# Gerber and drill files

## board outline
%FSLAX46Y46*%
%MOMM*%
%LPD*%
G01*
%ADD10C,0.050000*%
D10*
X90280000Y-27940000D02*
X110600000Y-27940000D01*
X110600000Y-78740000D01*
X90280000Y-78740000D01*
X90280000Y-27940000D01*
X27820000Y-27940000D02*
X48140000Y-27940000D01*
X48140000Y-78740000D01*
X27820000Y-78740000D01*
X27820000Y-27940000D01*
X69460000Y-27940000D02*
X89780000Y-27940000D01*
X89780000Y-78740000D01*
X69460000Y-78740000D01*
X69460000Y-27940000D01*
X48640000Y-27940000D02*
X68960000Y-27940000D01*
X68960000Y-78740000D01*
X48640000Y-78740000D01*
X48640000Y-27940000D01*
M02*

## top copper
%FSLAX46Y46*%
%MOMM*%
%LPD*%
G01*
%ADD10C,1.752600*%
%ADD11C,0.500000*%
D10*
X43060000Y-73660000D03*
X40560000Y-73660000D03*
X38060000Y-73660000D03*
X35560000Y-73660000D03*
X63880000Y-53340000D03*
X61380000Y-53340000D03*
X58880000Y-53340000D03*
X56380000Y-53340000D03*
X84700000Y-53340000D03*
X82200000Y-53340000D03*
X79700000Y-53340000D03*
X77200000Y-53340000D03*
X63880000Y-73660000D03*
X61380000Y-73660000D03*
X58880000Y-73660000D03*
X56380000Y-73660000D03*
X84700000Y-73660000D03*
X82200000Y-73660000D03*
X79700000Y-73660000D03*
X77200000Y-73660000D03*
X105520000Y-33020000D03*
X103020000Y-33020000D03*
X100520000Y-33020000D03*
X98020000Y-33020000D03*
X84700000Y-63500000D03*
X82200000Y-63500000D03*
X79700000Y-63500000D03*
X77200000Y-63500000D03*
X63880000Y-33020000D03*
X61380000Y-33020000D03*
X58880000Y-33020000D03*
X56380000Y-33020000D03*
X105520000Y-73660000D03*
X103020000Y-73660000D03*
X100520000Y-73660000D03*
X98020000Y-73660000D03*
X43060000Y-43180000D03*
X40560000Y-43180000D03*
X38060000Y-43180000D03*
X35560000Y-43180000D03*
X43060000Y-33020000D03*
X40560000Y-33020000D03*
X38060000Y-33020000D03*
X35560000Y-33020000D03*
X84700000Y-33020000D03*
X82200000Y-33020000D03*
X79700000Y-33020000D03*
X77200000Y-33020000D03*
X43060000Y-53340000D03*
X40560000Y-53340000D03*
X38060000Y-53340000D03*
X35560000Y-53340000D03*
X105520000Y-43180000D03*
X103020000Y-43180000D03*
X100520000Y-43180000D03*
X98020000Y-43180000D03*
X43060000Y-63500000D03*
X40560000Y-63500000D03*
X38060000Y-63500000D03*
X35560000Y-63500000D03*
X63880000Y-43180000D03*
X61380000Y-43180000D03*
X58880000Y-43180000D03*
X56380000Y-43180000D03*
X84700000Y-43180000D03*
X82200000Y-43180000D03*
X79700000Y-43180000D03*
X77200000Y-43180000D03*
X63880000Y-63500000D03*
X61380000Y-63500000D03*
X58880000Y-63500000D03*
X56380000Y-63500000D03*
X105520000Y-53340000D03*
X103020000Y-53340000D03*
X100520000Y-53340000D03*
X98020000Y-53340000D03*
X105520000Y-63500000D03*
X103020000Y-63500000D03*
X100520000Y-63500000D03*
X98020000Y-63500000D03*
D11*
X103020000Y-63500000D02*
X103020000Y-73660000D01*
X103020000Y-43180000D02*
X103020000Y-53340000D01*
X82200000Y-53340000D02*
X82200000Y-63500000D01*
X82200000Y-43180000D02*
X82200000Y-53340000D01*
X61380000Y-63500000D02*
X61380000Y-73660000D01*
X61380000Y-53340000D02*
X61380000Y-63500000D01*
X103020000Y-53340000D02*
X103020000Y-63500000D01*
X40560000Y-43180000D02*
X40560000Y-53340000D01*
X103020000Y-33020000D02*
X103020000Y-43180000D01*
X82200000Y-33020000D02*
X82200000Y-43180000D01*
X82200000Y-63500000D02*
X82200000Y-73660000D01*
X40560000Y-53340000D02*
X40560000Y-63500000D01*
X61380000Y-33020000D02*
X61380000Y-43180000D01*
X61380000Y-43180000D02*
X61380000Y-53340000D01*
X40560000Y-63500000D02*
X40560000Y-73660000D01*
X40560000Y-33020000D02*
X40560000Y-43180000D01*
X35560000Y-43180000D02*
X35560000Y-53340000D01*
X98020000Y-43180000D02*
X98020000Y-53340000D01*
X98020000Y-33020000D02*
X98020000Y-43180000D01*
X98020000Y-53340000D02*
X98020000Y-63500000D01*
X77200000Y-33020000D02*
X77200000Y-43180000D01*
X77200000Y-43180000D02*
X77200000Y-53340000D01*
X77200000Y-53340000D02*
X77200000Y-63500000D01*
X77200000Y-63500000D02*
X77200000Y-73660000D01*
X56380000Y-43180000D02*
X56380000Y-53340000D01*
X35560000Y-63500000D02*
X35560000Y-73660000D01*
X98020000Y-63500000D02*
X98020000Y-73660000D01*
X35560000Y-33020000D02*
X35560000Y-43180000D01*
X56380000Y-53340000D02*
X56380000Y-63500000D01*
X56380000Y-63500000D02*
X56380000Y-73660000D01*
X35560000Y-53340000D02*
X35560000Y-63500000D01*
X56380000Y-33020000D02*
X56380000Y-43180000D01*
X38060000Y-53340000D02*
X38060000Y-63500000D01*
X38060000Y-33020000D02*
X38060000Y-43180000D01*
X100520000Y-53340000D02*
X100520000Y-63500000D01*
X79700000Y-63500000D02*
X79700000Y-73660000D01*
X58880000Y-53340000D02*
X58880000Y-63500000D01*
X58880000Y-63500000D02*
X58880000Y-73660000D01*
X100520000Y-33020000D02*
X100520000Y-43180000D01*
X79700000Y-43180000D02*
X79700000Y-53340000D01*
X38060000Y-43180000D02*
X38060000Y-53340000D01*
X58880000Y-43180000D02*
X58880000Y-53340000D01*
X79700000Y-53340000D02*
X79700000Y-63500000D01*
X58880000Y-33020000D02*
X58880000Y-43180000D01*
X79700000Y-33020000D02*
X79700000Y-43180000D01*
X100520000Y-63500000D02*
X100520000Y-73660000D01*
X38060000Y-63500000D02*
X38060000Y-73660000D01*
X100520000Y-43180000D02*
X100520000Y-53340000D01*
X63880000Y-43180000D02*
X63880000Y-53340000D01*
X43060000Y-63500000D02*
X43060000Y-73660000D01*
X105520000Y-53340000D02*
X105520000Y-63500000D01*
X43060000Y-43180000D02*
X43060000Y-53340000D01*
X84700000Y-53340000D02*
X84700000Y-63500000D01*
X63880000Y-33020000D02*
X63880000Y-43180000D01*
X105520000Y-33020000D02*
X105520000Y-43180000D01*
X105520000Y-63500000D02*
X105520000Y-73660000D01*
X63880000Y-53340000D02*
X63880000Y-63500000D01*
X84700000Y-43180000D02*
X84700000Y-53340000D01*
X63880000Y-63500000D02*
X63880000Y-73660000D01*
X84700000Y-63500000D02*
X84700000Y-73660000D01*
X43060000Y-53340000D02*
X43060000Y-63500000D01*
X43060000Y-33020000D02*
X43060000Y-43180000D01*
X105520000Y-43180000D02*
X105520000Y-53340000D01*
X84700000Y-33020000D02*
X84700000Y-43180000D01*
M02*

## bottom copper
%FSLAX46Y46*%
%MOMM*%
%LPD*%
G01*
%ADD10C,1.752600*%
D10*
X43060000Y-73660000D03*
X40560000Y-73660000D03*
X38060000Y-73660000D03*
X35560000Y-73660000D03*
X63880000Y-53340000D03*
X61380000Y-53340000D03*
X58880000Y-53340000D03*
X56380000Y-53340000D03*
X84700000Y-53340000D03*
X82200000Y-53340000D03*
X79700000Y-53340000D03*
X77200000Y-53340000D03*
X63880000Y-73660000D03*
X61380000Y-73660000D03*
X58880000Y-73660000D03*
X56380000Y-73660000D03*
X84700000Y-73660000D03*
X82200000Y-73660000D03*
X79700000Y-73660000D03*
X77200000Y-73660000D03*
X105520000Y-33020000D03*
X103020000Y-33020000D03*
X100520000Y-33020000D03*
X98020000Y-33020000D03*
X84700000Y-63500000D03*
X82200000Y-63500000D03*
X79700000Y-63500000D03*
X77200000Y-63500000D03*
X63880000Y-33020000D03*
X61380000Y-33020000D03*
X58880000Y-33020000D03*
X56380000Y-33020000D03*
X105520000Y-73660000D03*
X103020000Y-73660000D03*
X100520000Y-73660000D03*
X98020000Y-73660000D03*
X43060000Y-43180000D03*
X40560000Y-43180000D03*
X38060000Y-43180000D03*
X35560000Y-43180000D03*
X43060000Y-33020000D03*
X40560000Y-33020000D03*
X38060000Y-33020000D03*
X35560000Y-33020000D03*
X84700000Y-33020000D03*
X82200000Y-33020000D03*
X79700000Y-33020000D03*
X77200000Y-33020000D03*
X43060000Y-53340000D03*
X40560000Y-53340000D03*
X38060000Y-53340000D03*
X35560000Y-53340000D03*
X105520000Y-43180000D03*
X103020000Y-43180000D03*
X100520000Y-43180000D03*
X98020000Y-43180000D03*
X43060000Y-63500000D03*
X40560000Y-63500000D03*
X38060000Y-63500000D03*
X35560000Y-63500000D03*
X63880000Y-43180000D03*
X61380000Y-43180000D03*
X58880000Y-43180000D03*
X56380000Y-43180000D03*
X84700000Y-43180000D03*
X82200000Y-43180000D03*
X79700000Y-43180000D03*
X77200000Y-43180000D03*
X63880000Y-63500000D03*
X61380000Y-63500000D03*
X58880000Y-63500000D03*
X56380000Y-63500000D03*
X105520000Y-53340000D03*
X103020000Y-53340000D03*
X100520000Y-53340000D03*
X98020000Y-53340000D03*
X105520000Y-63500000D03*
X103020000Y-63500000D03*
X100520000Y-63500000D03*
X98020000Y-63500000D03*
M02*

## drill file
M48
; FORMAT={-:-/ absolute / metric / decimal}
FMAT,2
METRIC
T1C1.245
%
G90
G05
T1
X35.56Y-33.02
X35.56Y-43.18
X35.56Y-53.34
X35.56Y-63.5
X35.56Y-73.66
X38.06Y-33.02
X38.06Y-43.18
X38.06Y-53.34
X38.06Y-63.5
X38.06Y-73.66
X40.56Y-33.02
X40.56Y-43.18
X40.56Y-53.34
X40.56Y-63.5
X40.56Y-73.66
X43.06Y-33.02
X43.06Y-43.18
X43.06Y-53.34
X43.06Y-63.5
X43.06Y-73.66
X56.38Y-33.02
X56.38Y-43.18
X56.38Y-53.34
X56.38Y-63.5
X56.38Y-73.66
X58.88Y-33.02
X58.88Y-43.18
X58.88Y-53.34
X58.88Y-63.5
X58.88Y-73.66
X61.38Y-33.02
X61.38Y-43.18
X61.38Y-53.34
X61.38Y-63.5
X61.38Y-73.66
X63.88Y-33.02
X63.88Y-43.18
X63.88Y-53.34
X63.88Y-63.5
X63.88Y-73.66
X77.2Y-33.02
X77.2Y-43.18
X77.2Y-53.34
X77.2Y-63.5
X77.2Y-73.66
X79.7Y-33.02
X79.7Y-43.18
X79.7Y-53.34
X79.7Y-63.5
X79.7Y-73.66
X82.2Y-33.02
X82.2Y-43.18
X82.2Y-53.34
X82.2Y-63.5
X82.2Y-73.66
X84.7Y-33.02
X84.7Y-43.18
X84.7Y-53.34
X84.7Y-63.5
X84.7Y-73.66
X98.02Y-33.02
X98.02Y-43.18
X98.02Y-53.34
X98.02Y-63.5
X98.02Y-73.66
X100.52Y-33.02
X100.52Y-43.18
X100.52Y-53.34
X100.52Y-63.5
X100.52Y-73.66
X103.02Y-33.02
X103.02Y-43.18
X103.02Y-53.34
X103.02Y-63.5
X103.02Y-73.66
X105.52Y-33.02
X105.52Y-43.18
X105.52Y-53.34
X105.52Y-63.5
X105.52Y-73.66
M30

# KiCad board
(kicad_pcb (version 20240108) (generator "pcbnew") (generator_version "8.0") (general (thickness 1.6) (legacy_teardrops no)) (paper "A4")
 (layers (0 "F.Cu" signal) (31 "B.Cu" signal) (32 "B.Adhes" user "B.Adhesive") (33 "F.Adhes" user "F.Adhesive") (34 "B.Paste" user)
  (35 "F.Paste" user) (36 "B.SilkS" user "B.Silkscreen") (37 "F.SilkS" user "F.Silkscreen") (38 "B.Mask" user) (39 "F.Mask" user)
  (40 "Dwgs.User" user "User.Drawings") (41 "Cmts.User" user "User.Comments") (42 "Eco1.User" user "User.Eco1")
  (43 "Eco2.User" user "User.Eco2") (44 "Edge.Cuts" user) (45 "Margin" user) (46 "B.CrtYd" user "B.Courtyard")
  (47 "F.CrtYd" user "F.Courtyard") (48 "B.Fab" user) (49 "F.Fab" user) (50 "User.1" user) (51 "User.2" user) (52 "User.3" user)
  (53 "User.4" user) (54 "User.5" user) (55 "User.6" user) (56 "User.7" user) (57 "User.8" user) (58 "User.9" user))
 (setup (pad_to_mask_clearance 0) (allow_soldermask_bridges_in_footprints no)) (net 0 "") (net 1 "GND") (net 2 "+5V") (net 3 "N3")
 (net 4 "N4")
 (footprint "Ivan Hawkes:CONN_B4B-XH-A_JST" (layer "F.Cu") (at 43.06 73.66)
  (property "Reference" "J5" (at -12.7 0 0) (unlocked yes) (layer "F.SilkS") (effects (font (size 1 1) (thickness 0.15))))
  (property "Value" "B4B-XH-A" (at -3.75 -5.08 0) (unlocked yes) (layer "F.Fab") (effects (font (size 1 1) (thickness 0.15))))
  (pad "1" thru_hole circle (at 0 0) (size 1.7526 1.7526) (drill 1.2446) (layers "*.Cu" "*.Mask") (remove_unused_layers no) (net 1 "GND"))
  (pad "2" thru_hole circle (at -2.5 0) (size 1.7526 1.7526) (drill 1.2446) (layers "*.Cu" "*.Mask") (remove_unused_layers no) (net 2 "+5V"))
  (pad "3" thru_hole circle (at -5 0) (size 1.7526 1.7526) (drill 1.2446) (layers "*.Cu" "*.Mask") (remove_unused_layers no) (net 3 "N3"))
  (pad "4" thru_hole circle (at -7.5 0) (size 1.7526 1.7526) (drill 1.2446) (layers "*.Cu" "*.Mask") (remove_unused_layers no) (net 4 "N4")))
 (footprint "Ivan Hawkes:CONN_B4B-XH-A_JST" (layer "F.Cu") (at 63.88 53.34)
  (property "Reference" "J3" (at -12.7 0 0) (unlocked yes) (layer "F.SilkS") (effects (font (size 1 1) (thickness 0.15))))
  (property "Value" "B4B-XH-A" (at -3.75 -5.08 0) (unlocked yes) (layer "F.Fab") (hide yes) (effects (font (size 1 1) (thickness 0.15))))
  (pad "1" thru_hole circle (at 0 0) (size 1.7526 1.7526) (drill 1.2446) (layers "*.Cu" "*.Mask") (remove_unused_layers no) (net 1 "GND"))
  (pad "2" thru_hole circle (at -2.5 0) (size 1.7526 1.7526) (drill 1.2446) (layers "*.Cu" "*.Mask") (remove_unused_layers no) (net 2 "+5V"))
  (pad "3" thru_hole circle (at -5 0) (size 1.7526 1.7526) (drill 1.2446) (layers "*.Cu" "*.Mask") (remove_unused_layers no) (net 3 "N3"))
  (pad "4" thru_hole circle (at -7.5 0) (size 1.7526 1.7526) (drill 1.2446) (layers "*.Cu" "*.Mask") (remove_unused_layers no) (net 4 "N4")))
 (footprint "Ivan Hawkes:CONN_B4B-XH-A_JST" (layer "F.Cu") (at 84.7 53.34)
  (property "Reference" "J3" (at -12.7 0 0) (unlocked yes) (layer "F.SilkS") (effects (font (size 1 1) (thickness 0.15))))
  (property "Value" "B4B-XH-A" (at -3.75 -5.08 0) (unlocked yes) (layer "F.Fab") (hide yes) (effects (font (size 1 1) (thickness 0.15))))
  (pad "1" thru_hole circle (at 0 0) (size 1.7526 1.7526) (drill 1.2446) (layers "*.Cu" "*.Mask") (remove_unused_layers no) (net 1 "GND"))
  (pad "2" thru_hole circle (at -2.5 0) (size 1.7526 1.7526) (drill 1.2446) (layers "*.Cu" "*.Mask") (remove_unused_layers no) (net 2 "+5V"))
  (pad "3" thru_hole circle (at -5 0) (size 1.7526 1.7526) (drill 1.2446) (layers "*.Cu" "*.Mask") (remove_unused_layers no) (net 3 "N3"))
  (pad "4" thru_hole circle (at -7.5 0) (size 1.7526 1.7526) (drill 1.2446) (layers "*.Cu" "*.Mask") (remove_unused_layers no) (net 4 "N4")))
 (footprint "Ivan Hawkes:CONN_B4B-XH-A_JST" (layer "F.Cu") (at 63.88 73.66)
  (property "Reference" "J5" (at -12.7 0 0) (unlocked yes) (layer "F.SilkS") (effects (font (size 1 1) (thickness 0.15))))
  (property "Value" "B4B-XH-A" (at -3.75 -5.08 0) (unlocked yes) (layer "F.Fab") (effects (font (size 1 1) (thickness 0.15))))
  (pad "1" thru_hole circle (at 0 0) (size 1.7526 1.7526) (drill 1.2446) (layers "*.Cu" "*.Mask") (remove_unused_layers no) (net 1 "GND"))
  (pad "2" thru_hole circle (at -2.5 0) (size 1.7526 1.7526) (drill 1.2446) (layers "*.Cu" "*.Mask") (remove_unused_layers no) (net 2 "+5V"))
  (pad "3" thru_hole circle (at -5 0) (size 1.7526 1.7526) (drill 1.2446) (layers "*.Cu" "*.Mask") (remove_unused_layers no) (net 3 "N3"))
  (pad "4" thru_hole circle (at -7.5 0) (size 1.7526 1.7526) (drill 1.2446) (layers "*.Cu" "*.Mask") (remove_unused_layers no) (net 4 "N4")))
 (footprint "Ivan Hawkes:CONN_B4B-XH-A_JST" (layer "F.Cu") (at 84.7 73.66)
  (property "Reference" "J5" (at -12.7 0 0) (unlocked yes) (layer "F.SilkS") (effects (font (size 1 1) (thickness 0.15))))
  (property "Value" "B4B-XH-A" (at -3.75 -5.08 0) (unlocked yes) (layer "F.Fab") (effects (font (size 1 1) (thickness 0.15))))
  (pad "1" thru_hole circle (at 0 0) (size 1.7526 1.7526) (drill 1.2446) (layers "*.Cu" "*.Mask") (remove_unused_layers no) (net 1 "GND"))
  (pad "2" thru_hole circle (at -2.5 0) (size 1.7526 1.7526) (drill 1.2446) (layers "*.Cu" "*.Mask") (remove_unused_layers no) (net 2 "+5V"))
  (pad "3" thru_hole circle (at -5 0) (size 1.7526 1.7526) (drill 1.2446) (layers "*.Cu" "*.Mask") (remove_unused_layers no) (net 3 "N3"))
  (pad "4" thru_hole circle (at -7.5 0) (size 1.7526 1.7526) (drill 1.2446) (layers "*.Cu" "*.Mask") (remove_unused_layers no) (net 4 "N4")))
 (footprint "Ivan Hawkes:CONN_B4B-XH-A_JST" (layer "F.Cu") (at 105.52 33.02)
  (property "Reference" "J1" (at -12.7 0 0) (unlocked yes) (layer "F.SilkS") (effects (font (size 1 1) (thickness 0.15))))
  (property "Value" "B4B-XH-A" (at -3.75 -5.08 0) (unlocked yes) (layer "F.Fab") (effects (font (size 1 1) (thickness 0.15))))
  (pad "1" thru_hole circle (at 0 0) (size 1.7526 1.7526) (drill 1.2446) (layers "*.Cu" "*.Mask") (remove_unused_layers no) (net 1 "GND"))
  (pad "2" thru_hole circle (at -2.5 0) (size 1.7526 1.7526) (drill 1.2446) (layers "*.Cu" "*.Mask") (remove_unused_layers no) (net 2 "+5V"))
  (pad "3" thru_hole circle (at -5 0) (size 1.7526 1.7526) (drill 1.2446) (layers "*.Cu" "*.Mask") (remove_unused_layers no) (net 3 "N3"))
  (pad "4" thru_hole circle (at -7.5 0) (size 1.7526 1.7526) (drill 1.2446) (layers "*.Cu" "*.Mask") (remove_unused_layers no) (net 4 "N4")))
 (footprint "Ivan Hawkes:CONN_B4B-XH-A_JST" (layer "F.Cu") (at 84.7 63.5)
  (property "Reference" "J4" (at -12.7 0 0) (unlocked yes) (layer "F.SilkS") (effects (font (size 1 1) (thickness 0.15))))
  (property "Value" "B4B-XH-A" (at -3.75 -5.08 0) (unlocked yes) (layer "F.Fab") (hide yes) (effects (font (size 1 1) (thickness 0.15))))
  (pad "1" thru_hole circle (at 0 0) (size 1.7526 1.7526) (drill 1.2446) (layers "*.Cu" "*.Mask") (remove_unused_layers no) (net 1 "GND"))
  (pad "2" thru_hole circle (at -2.5 0) (size 1.7526 1.7526) (drill 1.2446) (layers "*.Cu" "*.Mask") (remove_unused_layers no) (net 2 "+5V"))
  (pad "3" thru_hole circle (at -5 0) (size 1.7526 1.7526) (drill 1.2446) (layers "*.Cu" "*.Mask") (remove_unused_layers no) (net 3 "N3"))
  (pad "4" thru_hole circle (at -7.5 0) (size 1.7526 1.7526) (drill 1.2446) (layers "*.Cu" "*.Mask") (remove_unused_layers no) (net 4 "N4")))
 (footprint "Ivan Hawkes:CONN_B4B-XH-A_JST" (layer "F.Cu") (at 63.88 33.02)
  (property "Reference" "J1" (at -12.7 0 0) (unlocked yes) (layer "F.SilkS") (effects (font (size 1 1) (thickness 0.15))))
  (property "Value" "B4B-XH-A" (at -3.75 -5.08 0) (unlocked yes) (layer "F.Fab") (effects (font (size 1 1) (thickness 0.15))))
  (pad "1" thru_hole circle (at 0 0) (size 1.7526 1.7526) (drill 1.2446) (layers "*.Cu" "*.Mask") (remove_unused_layers no) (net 1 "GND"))
  (pad "2" thru_hole circle (at -2.5 0) (size 1.7526 1.7526) (drill 1.2446) (layers "*.Cu" "*.Mask") (remove_unused_layers no) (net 2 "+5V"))
  (pad "3" thru_hole circle (at -5 0) (size 1.7526 1.7526) (drill 1.2446) (layers "*.Cu" "*.Mask") (remove_unused_layers no) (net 3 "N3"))
  (pad "4" thru_hole circle (at -7.5 0) (size 1.7526 1.7526) (drill 1.2446) (layers "*.Cu" "*.Mask") (remove_unused_layers no) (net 4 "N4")))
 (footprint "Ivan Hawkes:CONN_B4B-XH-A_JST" (layer "F.Cu") (at 105.52 73.66)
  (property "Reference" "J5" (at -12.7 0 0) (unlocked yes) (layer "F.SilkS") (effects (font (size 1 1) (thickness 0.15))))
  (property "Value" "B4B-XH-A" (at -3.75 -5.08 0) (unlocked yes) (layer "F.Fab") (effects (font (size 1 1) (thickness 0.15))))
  (pad "1" thru_hole circle (at 0 0) (size 1.7526 1.7526) (drill 1.2446) (layers "*.Cu" "*.Mask") (remove_unused_layers no) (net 1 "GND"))
  (pad "2" thru_hole circle (at -2.5 0) (size 1.7526 1.7526) (drill 1.2446) (layers "*.Cu" "*.Mask") (remove_unused_layers no) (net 2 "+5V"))
  (pad "3" thru_hole circle (at -5 0) (size 1.7526 1.7526) (drill 1.2446) (layers "*.Cu" "*.Mask") (remove_unused_layers no) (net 3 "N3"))
  (pad "4" thru_hole circle (at -7.5 0) (size 1.7526 1.7526) (drill 1.2446) (layers "*.Cu" "*.Mask") (remove_unused_layers no) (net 4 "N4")))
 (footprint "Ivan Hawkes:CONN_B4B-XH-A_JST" (layer "F.Cu") (at 43.06 43.18)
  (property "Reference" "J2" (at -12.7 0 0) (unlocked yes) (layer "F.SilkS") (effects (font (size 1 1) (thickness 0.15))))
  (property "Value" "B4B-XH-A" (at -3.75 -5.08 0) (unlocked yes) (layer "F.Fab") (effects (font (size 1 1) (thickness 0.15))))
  (pad "1" thru_hole circle (at 0 0) (size 1.7526 1.7526) (drill 1.2446) (layers "*.Cu" "*.Mask") (remove_unused_layers no) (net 1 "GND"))
  (pad "2" thru_hole circle (at -2.5 0) (size 1.7526 1.7526) (drill 1.2446) (layers "*.Cu" "*.Mask") (remove_unused_layers no) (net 2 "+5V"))
  (pad "3" thru_hole circle (at -5 0) (size 1.7526 1.7526) (drill 1.2446) (layers "*.Cu" "*.Mask") (remove_unused_layers no) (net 3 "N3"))
  (pad "4" thru_hole circle (at -7.5 0) (size 1.7526 1.7526) (drill 1.2446) (layers "*.Cu" "*.Mask") (remove_unused_layers no) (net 4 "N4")))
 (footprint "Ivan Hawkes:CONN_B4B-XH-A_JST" (layer "F.Cu") (at 43.06 33.02)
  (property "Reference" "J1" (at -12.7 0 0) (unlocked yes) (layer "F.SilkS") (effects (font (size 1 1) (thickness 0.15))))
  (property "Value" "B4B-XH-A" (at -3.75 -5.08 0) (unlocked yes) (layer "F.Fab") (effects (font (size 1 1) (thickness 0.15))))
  (pad "1" thru_hole circle (at 0 0) (size 1.7526 1.7526) (drill 1.2446) (layers "*.Cu" "*.Mask") (remove_unused_layers no) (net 1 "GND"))
  (pad "2" thru_hole circle (at -2.5 0) (size 1.7526 1.7526) (drill 1.2446) (layers "*.Cu" "*.Mask") (remove_unused_layers no) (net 2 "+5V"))
  (pad "3" thru_hole circle (at -5 0) (size 1.7526 1.7526) (drill 1.2446) (layers "*.Cu" "*.Mask") (remove_unused_layers no) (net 3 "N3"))
  (pad "4" thru_hole circle (at -7.5 0) (size 1.7526 1.7526) (drill 1.2446) (layers "*.Cu" "*.Mask") (remove_unused_layers no) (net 4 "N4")))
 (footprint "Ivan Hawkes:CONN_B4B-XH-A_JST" (layer "F.Cu") (at 84.7 33.02)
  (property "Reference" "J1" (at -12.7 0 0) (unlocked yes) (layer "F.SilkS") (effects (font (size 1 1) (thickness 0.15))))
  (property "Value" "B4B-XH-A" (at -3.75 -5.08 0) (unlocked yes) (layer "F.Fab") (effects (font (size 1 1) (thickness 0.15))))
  (pad "1" thru_hole circle (at 0 0) (size 1.7526 1.7526) (drill 1.2446) (layers "*.Cu" "*.Mask") (remove_unused_layers no) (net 1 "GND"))
  (pad "2" thru_hole circle (at -2.5 0) (size 1.7526 1.7526) (drill 1.2446) (layers "*.Cu" "*.Mask") (remove_unused_layers no) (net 2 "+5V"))
  (pad "3" thru_hole circle (at -5 0) (size 1.7526 1.7526) (drill 1.2446) (layers "*.Cu" "*.Mask") (remove_unused_layers no) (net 3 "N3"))
  (pad "4" thru_hole circle (at -7.5 0) (size 1.7526 1.7526) (drill 1.2446) (layers "*.Cu" "*.Mask") (remove_unused_layers no) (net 4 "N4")))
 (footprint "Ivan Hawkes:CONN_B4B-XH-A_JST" (layer "F.Cu") (at 43.06 53.34)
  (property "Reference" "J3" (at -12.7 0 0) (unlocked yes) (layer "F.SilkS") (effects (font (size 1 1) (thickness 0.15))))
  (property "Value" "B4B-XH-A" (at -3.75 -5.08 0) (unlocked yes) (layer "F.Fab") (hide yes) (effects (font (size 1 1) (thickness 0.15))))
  (pad "1" thru_hole circle (at 0 0) (size 1.7526 1.7526) (drill 1.2446) (layers "*.Cu" "*.Mask") (remove_unused_layers no) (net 1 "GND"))
  (pad "2" thru_hole circle (at -2.5 0) (size 1.7526 1.7526) (drill 1.2446) (layers "*.Cu" "*.Mask") (remove_unused_layers no) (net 2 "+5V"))
  (pad "3" thru_hole circle (at -5 0) (size 1.7526 1.7526) (drill 1.2446) (layers "*.Cu" "*.Mask") (remove_unused_layers no) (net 3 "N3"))
  (pad "4" thru_hole circle (at -7.5 0) (size 1.7526 1.7526) (drill 1.2446) (layers "*.Cu" "*.Mask") (remove_unused_layers no) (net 4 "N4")))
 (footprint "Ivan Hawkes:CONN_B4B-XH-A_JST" (layer "F.Cu") (at 105.52 43.18)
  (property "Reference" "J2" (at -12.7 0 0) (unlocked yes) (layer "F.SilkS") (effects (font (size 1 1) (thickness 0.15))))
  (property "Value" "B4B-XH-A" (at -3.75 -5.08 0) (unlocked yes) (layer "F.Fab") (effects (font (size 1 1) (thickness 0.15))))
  (pad "1" thru_hole circle (at 0 0) (size 1.7526 1.7526) (drill 1.2446) (layers "*.Cu" "*.Mask") (remove_unused_layers no) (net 1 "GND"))
  (pad "2" thru_hole circle (at -2.5 0) (size 1.7526 1.7526) (drill 1.2446) (layers "*.Cu" "*.Mask") (remove_unused_layers no) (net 2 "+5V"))
  (pad "3" thru_hole circle (at -5 0) (size 1.7526 1.7526) (drill 1.2446) (layers "*.Cu" "*.Mask") (remove_unused_layers no) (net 3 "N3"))
  (pad "4" thru_hole circle (at -7.5 0) (size 1.7526 1.7526) (drill 1.2446) (layers "*.Cu" "*.Mask") (remove_unused_layers no) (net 4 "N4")))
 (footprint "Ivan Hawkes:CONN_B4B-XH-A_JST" (layer "F.Cu") (at 43.06 63.5)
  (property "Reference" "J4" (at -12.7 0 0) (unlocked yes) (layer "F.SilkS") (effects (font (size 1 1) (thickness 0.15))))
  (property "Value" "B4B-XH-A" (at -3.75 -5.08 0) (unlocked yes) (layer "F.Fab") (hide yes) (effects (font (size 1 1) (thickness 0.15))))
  (pad "1" thru_hole circle (at 0 0) (size 1.7526 1.7526) (drill 1.2446) (layers "*.Cu" "*.Mask") (remove_unused_layers no) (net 1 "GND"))
  (pad "2" thru_hole circle (at -2.5 0) (size 1.7526 1.7526) (drill 1.2446) (layers "*.Cu" "*.Mask") (remove_unused_layers no) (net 2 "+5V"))
  (pad "3" thru_hole circle (at -5 0) (size 1.7526 1.7526) (drill 1.2446) (layers "*.Cu" "*.Mask") (remove_unused_layers no) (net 3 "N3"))
  (pad "4" thru_hole circle (at -7.5 0) (size 1.7526 1.7526) (drill 1.2446) (layers "*.Cu" "*.Mask") (remove_unused_layers no) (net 4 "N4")))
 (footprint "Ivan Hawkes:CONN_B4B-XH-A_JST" (layer "F.Cu") (at 63.88 43.18)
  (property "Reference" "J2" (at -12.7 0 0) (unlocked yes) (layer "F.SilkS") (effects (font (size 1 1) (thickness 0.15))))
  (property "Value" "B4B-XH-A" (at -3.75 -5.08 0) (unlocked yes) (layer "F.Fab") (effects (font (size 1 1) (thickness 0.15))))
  (pad "1" thru_hole circle (at 0 0) (size 1.7526 1.7526) (drill 1.2446) (layers "*.Cu" "*.Mask") (remove_unused_layers no) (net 1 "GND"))
  (pad "2" thru_hole circle (at -2.5 0) (size 1.7526 1.7526) (drill 1.2446) (layers "*.Cu" "*.Mask") (remove_unused_layers no) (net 2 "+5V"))
  (pad "3" thru_hole circle (at -5 0) (size 1.7526 1.7526) (drill 1.2446) (layers "*.Cu" "*.Mask") (remove_unused_layers no) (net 3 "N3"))
  (pad "4" thru_hole circle (at -7.5 0) (size 1.7526 1.7526) (drill 1.2446) (layers "*.Cu" "*.Mask") (remove_unused_layers no) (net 4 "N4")))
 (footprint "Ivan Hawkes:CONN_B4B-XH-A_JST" (layer "F.Cu") (at 84.7 43.18)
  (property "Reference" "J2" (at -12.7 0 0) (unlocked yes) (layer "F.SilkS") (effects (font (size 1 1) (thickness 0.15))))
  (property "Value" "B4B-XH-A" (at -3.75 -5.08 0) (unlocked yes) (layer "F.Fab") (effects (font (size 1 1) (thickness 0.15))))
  (pad "1" thru_hole circle (at 0 0) (size 1.7526 1.7526) (drill 1.2446) (layers "*.Cu" "*.Mask") (remove_unused_layers no) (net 1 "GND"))
  (pad "2" thru_hole circle (at -2.5 0) (size 1.7526 1.7526) (drill 1.2446) (layers "*.Cu" "*.Mask") (remove_unused_layers no) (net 2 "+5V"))
  (pad "3" thru_hole circle (at -5 0) (size 1.7526 1.7526) (drill 1.2446) (layers "*.Cu" "*.Mask") (remove_unused_layers no) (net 3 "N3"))
  (pad "4" thru_hole circle (at -7.5 0) (size 1.7526 1.7526) (drill 1.2446) (layers "*.Cu" "*.Mask") (remove_unused_layers no) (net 4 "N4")))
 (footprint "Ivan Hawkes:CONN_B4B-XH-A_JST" (layer "F.Cu") (at 63.88 63.5)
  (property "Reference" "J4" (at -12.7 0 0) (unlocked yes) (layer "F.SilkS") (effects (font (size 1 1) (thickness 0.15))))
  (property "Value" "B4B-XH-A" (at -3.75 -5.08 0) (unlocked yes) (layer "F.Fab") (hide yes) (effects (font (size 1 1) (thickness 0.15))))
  (pad "1" thru_hole circle (at 0 0) (size 1.7526 1.7526) (drill 1.2446) (layers "*.Cu" "*.Mask") (remove_unused_layers no) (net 1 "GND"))
  (pad "2" thru_hole circle (at -2.5 0) (size 1.7526 1.7526) (drill 1.2446) (layers "*.Cu" "*.Mask") (remove_unused_layers no) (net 2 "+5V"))
  (pad "3" thru_hole circle (at -5 0) (size 1.7526 1.7526) (drill 1.2446) (layers "*.Cu" "*.Mask") (remove_unused_layers no) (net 3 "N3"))
  (pad "4" thru_hole circle (at -7.5 0) (size 1.7526 1.7526) (drill 1.2446) (layers "*.Cu" "*.Mask") (remove_unused_layers no) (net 4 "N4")))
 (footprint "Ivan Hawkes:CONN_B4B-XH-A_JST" (layer "F.Cu") (at 105.52 53.34)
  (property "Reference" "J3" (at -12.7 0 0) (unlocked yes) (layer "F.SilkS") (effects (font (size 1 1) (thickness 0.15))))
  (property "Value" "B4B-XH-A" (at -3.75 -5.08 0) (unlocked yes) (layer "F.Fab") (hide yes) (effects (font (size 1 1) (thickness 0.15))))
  (pad "1" thru_hole circle (at 0 0) (size 1.7526 1.7526) (drill 1.2446) (layers "*.Cu" "*.Mask") (remove_unused_layers no) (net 1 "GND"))
  (pad "2" thru_hole circle (at -2.5 0) (size 1.7526 1.7526) (drill 1.2446) (layers "*.Cu" "*.Mask") (remove_unused_layers no) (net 2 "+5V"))
  (pad "3" thru_hole circle (at -5 0) (size 1.7526 1.7526) (drill 1.2446) (layers "*.Cu" "*.Mask") (remove_unused_layers no) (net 3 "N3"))
  (pad "4" thru_hole circle (at -7.5 0) (size 1.7526 1.7526) (drill 1.2446) (layers "*.Cu" "*.Mask") (remove_unused_layers no) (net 4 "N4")))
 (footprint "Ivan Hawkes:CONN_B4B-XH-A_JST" (layer "F.Cu") (at 105.52 63.5)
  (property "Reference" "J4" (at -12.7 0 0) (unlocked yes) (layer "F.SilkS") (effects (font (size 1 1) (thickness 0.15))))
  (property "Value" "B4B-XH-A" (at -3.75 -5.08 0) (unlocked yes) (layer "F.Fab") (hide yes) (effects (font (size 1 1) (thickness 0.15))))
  (pad "1" thru_hole circle (at 0 0) (size 1.7526 1.7526) (drill 1.2446) (layers "*.Cu" "*.Mask") (remove_unused_layers no) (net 1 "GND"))
  (pad "2" thru_hole circle (at -2.5 0) (size 1.7526 1.7526) (drill 1.2446) (layers "*.Cu" "*.Mask") (remove_unused_layers no) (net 2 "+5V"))
  (pad "3" thru_hole circle (at -5 0) (size 1.7526 1.7526) (drill 1.2446) (layers "*.Cu" "*.Mask") (remove_unused_layers no) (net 3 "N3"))
  (pad "4" thru_hole circle (at -7.5 0) (size 1.7526 1.7526) (drill 1.2446) (layers "*.Cu" "*.Mask") (remove_unused_layers no) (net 4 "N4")))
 (gr_rect (start 90.28 27.94) (end 110.6 78.74) (stroke (width 0.05) (type default)) (fill none) (layer "Edge.Cuts"))
 (gr_rect (start 27.82 27.94) (end 48.14 78.74) (stroke (width 0.05) (type default)) (fill none) (layer "Edge.Cuts"))
 (gr_rect (start 69.46 27.94) (end 89.78 78.74) (stroke (width 0.05) (type default)) (fill none) (layer "Edge.Cuts"))
 (gr_rect (start 48.64 27.94) (end 68.96 78.74) (stroke (width 0.05) (type default)) (fill none) (layer "Edge.Cuts"))
 (segment (start 103.02 63.5) (end 103.02 73.66) (width 0.5) (layer "F.Cu") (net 2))
 (segment (start 103.02 43.18) (end 103.02 53.34) (width 0.5) (layer "F.Cu") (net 2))
 (segment (start 82.2 53.34) (end 82.2 63.5) (width 0.5) (layer "F.Cu") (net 2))
 (segment (start 82.2 43.18) (end 82.2 53.34) (width 0.5) (layer "F.Cu") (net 2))
 (segment (start 61.38 63.5) (end 61.38 73.66) (width 0.5) (layer "F.Cu") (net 2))
 (segment (start 61.38 53.34) (end 61.38 63.5) (width 0.5) (layer "F.Cu") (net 2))
 (segment (start 103.02 53.34) (end 103.02 63.5) (width 0.5) (layer "F.Cu") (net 2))
 (segment (start 40.56 43.18) (end 40.56 53.34) (width 0.5) (layer "F.Cu") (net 2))
 (segment (start 103.02 33.02) (end 103.02 43.18) (width 0.5) (layer "F.Cu") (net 2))
 (segment (start 82.2 33.02) (end 82.2 43.18) (width 0.5) (layer "F.Cu") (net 2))
 (segment (start 82.2 63.5) (end 82.2 73.66) (width 0.5) (layer "F.Cu") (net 2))
 (segment (start 40.56 53.34) (end 40.56 63.5) (width 0.5) (layer "F.Cu") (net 2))
 (segment (start 61.38 33.02) (end 61.38 43.18) (width 0.5) (layer "F.Cu") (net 2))
 (segment (start 61.38 43.18) (end 61.38 53.34) (width 0.5) (layer "F.Cu") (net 2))
 (segment (start 40.56 63.5) (end 40.56 73.66) (width 0.5) (layer "F.Cu") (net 2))
 (segment (start 40.56 33.02) (end 40.56 43.18) (width 0.5) (layer "F.Cu") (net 2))
 (segment (start 35.56 43.18) (end 35.56 53.34) (width 0.5) (layer "F.Cu") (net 4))
 (segment (start 98.02 43.18) (end 98.02 53.34) (width 0.5) (layer "F.Cu") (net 4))
 (segment (start 98.02 33.02) (end 98.02 43.18) (width 0.5) (layer "F.Cu") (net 4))
 (segment (start 98.02 53.34) (end 98.02 63.5) (width 0.5) (layer "F.Cu") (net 4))
 (segment (start 77.2 33.02) (end 77.2 43.18) (width 0.5) (layer "F.Cu") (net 4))
 (segment (start 77.2 43.18) (end 77.2 53.34) (width 0.5) (layer "F.Cu") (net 4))
 (segment (start 77.2 53.34) (end 77.2 63.5) (width 0.5) (layer "F.Cu") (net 4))
 (segment (start 77.2 63.5) (end 77.2 73.66) (width 0.5) (layer "F.Cu") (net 4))
 (segment (start 56.38 43.18) (end 56.38 53.34) (width 0.5) (layer "F.Cu") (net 4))
 (segment (start 35.56 63.5) (end 35.56 73.66) (width 0.5) (layer "F.Cu") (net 4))
 (segment (start 98.02 63.5) (end 98.02 73.66) (width 0.5) (layer "F.Cu") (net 4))
 (segment (start 35.56 33.02) (end 35.56 43.18) (width 0.5) (layer "F.Cu") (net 4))
 (segment (start 56.38 53.34) (end 56.38 63.5) (width 0.5) (layer "F.Cu") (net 4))
 (segment (start 56.38 63.5) (end 56.38 73.66) (width 0.5) (layer "F.Cu") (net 4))
 (segment (start 35.56 53.34) (end 35.56 63.5) (width 0.5) (layer "F.Cu") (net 4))
 (segment (start 56.38 33.02) (end 56.38 43.18) (width 0.5) (layer "F.Cu") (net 4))
 (segment (start 38.06 53.34) (end 38.06 63.5) (width 0.5) (layer "F.Cu") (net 3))
 (segment (start 38.06 33.02) (end 38.06 43.18) (width 0.5) (layer "F.Cu") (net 3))
 (segment (start 100.52 53.34) (end 100.52 63.5) (width 0.5) (layer "F.Cu") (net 3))
 (segment (start 79.7 63.5) (end 79.7 73.66) (width 0.5) (layer "F.Cu") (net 3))
 (segment (start 58.88 53.34) (end 58.88 63.5) (width 0.5) (layer "F.Cu") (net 3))
 (segment (start 58.88 63.5) (end 58.88 73.66) (width 0.5) (layer "F.Cu") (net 3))
 (segment (start 100.52 33.02) (end 100.52 43.18) (width 0.5) (layer "F.Cu") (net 3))
 (segment (start 79.7 43.18) (end 79.7 53.34) (width 0.5) (layer "F.Cu") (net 3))
 (segment (start 38.06 43.18) (end 38.06 53.34) (width 0.5) (layer "F.Cu") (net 3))
 (segment (start 58.88 43.18) (end 58.88 53.34) (width 0.5) (layer "F.Cu") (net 3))
 (segment (start 79.7 53.34) (end 79.7 63.5) (width 0.5) (layer "F.Cu") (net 3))
 (segment (start 58.88 33.02) (end 58.88 43.18) (width 0.5) (layer "F.Cu") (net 3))
 (segment (start 79.7 33.02) (end 79.7 43.18) (width 0.5) (layer "F.Cu") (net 3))
 (segment (start 100.52 63.5) (end 100.52 73.66) (width 0.5) (layer "F.Cu") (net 3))
 (segment (start 38.06 63.5) (end 38.06 73.66) (width 0.5) (layer "F.Cu") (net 3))
 (segment (start 100.52 43.18) (end 100.52 53.34) (width 0.5) (layer "F.Cu") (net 3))
 (segment (start 63.88 43.18) (end 63.88 53.34) (width 0.5) (layer "F.Cu") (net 1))
 (segment (start 43.06 63.5) (end 43.06 73.66) (width 0.5) (layer "F.Cu") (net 1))
 (segment (start 105.52 53.34) (end 105.52 63.5) (width 0.5) (layer "F.Cu") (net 1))
 (segment (start 43.06 43.18) (end 43.06 53.34) (width 0.5) (layer "F.Cu") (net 1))
 (segment (start 84.7 53.34) (end 84.7 63.5) (width 0.5) (layer "F.Cu") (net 1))
 (segment (start 63.88 33.02) (end 63.88 43.18) (width 0.5) (layer "F.Cu") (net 1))
 (segment (start 105.52 33.02) (end 105.52 43.18) (width 0.5) (layer "F.Cu") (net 1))
 (segment (start 105.52 63.5) (end 105.52 73.66) (width 0.5) (layer "F.Cu") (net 1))
 (segment (start 63.88 53.34) (end 63.88 63.5) (width 0.5) (layer "F.Cu") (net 1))
 (segment (start 84.7 43.18) (end 84.7 53.34) (width 0.5) (layer "F.Cu") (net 1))
 (segment (start 63.88 63.5) (end 63.88 73.66) (width 0.5) (layer "F.Cu") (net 1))
 (segment (start 84.7 63.5) (end 84.7 73.66) (width 0.5) (layer "F.Cu") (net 1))
 (segment (start 43.06 53.34) (end 43.06 63.5) (width 0.5) (layer "F.Cu") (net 1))
 (segment (start 43.06 33.02) (end 43.06 43.18) (width 0.5) (layer "F.Cu") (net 1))
 (segment (start 105.52 43.18) (end 105.52 53.34) (width 0.5) (layer "F.Cu") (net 1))
 (segment (start 84.7 33.02) (end 84.7 43.18) (width 0.5) (layer "F.Cu") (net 1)))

